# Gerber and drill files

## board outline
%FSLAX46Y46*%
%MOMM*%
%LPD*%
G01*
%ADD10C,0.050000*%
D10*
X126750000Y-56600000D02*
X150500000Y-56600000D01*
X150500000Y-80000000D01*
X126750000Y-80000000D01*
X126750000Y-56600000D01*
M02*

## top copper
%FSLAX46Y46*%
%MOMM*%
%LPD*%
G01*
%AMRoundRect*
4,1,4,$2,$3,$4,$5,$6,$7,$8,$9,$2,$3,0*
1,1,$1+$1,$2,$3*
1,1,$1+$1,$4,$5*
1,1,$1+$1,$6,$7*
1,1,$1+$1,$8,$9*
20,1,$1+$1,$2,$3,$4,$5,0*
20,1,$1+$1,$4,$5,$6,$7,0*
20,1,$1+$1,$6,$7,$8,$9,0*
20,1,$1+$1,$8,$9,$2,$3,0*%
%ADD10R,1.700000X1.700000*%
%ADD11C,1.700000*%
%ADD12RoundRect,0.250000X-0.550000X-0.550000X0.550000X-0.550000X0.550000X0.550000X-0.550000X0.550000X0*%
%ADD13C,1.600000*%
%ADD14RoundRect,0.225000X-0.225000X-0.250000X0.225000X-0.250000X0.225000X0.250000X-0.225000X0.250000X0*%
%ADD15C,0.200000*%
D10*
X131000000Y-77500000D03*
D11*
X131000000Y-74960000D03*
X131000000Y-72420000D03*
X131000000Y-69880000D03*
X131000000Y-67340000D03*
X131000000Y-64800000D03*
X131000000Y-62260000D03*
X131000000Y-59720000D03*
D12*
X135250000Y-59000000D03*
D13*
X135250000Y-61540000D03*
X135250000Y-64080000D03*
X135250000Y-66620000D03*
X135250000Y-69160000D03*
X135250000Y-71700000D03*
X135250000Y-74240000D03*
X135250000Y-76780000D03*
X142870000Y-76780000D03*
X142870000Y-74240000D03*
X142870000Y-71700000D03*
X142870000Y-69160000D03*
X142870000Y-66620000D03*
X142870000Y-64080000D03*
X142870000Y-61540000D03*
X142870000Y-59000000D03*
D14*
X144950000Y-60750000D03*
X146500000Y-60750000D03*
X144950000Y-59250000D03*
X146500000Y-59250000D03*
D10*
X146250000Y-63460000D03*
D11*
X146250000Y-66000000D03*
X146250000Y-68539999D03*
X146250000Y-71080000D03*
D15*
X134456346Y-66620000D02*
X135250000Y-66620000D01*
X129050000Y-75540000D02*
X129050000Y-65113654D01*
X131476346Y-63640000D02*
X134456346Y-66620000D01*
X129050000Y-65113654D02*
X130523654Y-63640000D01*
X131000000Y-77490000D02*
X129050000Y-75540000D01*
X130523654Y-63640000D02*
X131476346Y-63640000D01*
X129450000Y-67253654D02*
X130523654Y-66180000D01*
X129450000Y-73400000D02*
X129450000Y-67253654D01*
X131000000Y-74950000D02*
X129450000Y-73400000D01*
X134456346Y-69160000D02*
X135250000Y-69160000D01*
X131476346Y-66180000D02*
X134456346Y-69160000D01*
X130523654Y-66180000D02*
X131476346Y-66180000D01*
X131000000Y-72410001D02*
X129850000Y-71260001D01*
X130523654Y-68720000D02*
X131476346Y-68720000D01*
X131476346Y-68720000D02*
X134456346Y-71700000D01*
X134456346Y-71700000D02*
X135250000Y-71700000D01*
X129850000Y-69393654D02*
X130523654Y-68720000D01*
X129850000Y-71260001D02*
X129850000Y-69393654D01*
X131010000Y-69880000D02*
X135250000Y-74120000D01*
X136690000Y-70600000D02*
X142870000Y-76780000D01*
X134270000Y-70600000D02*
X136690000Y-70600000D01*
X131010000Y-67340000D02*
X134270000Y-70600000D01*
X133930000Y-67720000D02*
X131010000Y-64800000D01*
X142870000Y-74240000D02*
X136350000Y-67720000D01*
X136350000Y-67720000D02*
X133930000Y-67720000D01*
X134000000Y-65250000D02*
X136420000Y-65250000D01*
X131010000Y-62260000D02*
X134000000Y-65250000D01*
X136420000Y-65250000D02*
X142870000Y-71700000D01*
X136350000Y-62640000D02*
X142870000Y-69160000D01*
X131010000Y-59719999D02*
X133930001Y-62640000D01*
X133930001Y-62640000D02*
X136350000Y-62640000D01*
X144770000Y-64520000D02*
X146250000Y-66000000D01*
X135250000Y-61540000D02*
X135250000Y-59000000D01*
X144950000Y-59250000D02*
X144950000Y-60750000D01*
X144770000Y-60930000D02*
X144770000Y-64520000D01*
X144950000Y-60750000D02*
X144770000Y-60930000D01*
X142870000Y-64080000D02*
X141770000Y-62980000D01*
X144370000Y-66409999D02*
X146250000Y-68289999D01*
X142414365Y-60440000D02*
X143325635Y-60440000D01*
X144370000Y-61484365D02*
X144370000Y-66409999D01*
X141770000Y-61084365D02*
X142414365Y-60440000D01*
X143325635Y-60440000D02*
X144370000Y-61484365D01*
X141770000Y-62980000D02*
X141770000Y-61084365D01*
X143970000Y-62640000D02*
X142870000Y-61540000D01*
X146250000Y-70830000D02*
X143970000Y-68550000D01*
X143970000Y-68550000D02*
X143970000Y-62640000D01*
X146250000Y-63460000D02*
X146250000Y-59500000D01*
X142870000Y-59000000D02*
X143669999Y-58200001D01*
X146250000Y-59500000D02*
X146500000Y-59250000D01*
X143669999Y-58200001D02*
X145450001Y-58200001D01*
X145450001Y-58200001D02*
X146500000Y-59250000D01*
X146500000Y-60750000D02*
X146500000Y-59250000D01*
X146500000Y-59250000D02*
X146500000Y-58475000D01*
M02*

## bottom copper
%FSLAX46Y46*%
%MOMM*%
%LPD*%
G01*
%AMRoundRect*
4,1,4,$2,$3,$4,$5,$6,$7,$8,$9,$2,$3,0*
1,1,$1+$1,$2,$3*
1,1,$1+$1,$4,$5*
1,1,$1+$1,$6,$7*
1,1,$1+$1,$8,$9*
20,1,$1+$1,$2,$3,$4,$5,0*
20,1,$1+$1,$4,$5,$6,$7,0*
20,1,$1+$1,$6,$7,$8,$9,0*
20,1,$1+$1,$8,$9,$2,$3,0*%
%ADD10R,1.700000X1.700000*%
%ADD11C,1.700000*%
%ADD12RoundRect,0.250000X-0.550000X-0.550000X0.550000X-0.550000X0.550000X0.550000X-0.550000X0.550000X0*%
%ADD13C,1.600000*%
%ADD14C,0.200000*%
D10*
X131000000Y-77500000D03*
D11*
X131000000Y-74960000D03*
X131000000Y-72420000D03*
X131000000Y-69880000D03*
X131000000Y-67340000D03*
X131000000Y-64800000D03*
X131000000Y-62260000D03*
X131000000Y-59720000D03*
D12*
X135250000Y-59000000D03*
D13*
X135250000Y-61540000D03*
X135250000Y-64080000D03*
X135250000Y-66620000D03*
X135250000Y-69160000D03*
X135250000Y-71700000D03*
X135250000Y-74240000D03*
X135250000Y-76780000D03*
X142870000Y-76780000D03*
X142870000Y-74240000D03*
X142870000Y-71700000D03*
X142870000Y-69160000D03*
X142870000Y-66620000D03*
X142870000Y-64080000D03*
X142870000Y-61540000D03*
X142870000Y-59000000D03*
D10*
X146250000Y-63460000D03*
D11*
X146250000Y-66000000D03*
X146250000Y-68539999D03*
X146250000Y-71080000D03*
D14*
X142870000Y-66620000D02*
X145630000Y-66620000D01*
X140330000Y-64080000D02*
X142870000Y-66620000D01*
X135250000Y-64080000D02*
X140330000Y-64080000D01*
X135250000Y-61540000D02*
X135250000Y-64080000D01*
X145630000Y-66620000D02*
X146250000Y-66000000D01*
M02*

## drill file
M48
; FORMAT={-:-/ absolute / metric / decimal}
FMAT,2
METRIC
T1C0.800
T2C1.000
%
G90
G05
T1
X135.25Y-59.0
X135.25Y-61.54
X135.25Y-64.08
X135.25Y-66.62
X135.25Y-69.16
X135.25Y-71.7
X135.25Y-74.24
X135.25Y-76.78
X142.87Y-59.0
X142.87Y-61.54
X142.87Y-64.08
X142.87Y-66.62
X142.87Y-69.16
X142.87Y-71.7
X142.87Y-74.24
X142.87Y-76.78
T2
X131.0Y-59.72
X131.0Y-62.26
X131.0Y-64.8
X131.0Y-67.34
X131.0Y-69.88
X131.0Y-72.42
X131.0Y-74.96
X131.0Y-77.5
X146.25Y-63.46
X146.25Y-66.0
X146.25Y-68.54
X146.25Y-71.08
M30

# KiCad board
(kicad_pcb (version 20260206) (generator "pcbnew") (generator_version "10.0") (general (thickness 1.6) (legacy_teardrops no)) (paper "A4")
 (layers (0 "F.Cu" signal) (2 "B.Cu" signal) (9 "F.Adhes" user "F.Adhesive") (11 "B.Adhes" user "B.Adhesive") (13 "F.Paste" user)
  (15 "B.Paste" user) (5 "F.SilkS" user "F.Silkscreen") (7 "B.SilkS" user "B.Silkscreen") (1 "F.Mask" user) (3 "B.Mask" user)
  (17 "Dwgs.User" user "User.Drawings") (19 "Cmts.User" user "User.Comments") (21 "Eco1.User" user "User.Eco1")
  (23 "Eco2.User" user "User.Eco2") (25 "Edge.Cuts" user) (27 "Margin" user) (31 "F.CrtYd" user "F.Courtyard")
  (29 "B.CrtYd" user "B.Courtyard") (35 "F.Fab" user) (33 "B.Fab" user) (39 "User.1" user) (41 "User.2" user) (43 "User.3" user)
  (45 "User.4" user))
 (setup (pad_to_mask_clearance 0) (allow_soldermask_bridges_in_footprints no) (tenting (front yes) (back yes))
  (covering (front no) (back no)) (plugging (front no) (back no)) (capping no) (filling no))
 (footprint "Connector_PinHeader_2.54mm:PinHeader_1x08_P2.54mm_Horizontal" (layer "F.Cu") (at 131 77.5 180)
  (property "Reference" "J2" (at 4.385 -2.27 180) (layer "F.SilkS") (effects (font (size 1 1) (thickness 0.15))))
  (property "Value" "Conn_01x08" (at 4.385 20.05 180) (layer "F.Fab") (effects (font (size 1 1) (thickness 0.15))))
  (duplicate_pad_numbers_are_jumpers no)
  (pad "1" thru_hole rect (at 0 0 180) (size 1.7 1.7) (drill 1) (layers "*.Cu" "*.Mask") (remove_unused_layers no) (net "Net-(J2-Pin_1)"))
  (pad "2" thru_hole circle (at 0 2.54 180) (size 1.7 1.7) (drill 1) (layers "*.Cu" "*.Mask") (remove_unused_layers no)
   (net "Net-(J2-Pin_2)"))
  (pad "3" thru_hole circle (at 0 5.08 180) (size 1.7 1.7) (drill 1) (layers "*.Cu" "*.Mask") (remove_unused_layers no)
   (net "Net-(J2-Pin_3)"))
  (pad "4" thru_hole circle (at 0 7.62 180) (size 1.7 1.7) (drill 1) (layers "*.Cu" "*.Mask") (remove_unused_layers no)
   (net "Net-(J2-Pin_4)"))
  (pad "5" thru_hole circle (at 0 10.16 180) (size 1.7 1.7) (drill 1) (layers "*.Cu" "*.Mask") (remove_unused_layers no)
   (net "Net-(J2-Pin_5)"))
  (pad "6" thru_hole circle (at 0 12.7 180) (size 1.7 1.7) (drill 1) (layers "*.Cu" "*.Mask") (remove_unused_layers no)
   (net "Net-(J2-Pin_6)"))
  (pad "7" thru_hole circle (at 0 15.24 180) (size 1.7 1.7) (drill 1) (layers "*.Cu" "*.Mask") (remove_unused_layers no)
   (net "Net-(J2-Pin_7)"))
  (pad "8" thru_hole circle (at 0 17.78 180) (size 1.7 1.7) (drill 1) (layers "*.Cu" "*.Mask") (remove_unused_layers no)
   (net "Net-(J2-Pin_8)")))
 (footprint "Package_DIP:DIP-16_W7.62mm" (layer "F.Cu") (at 135.25 59)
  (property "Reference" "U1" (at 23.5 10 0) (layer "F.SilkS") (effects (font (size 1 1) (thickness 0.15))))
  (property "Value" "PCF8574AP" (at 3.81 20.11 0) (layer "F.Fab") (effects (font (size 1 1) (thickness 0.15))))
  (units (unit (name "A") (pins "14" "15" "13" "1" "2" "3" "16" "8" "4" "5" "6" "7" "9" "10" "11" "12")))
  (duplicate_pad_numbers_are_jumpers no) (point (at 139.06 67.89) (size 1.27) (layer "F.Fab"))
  (pad "1" thru_hole roundrect (at 0 0) (size 1.6 1.6) (drill 0.8) (layers "*.Cu" "*.Mask") (remove_unused_layers no)
   (roundrect_rratio 0.15625) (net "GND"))
  (pad "2" thru_hole circle (at 0 2.54) (size 1.6 1.6) (drill 0.8) (layers "*.Cu" "*.Mask") (remove_unused_layers no) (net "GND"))
  (pad "3" thru_hole circle (at 0 5.08) (size 1.6 1.6) (drill 0.8) (layers "*.Cu" "*.Mask") (remove_unused_layers no) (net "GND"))
  (pad "4" thru_hole circle (at 0 7.62) (size 1.6 1.6) (drill 0.8) (layers "*.Cu" "*.Mask") (remove_unused_layers no) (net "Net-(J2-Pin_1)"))
  (pad "5" thru_hole circle (at 0 10.16) (size 1.6 1.6) (drill 0.8) (layers "*.Cu" "*.Mask") (remove_unused_layers no)
   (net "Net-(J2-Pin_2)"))
  (pad "6" thru_hole circle (at 0 12.7) (size 1.6 1.6) (drill 0.8) (layers "*.Cu" "*.Mask") (remove_unused_layers no) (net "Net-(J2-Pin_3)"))
  (pad "7" thru_hole circle (at 0 15.24) (size 1.6 1.6) (drill 0.8) (layers "*.Cu" "*.Mask") (remove_unused_layers no)
   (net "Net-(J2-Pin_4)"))
  (pad "8" thru_hole circle (at 0 17.78) (size 1.6 1.6) (drill 0.8) (layers "*.Cu" "*.Mask") (remove_unused_layers no)
   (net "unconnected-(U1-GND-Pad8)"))
  (pad "9" thru_hole circle (at 7.62 17.78) (size 1.6 1.6) (drill 0.8) (layers "*.Cu" "*.Mask") (remove_unused_layers no)
   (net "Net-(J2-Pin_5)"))
  (pad "10" thru_hole circle (at 7.62 15.24) (size 1.6 1.6) (drill 0.8) (layers "*.Cu" "*.Mask") (remove_unused_layers no)
   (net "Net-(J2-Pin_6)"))
  (pad "11" thru_hole circle (at 7.62 12.7) (size 1.6 1.6) (drill 0.8) (layers "*.Cu" "*.Mask") (remove_unused_layers no)
   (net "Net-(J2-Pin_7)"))
  (pad "12" thru_hole circle (at 7.62 10.16) (size 1.6 1.6) (drill 0.8) (layers "*.Cu" "*.Mask") (remove_unused_layers no)
   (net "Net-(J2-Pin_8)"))
  (pad "13" thru_hole circle (at 7.62 7.62) (size 1.6 1.6) (drill 0.8) (layers "*.Cu" "*.Mask") (remove_unused_layers no) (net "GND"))
  (pad "14" thru_hole circle (at 7.62 5.08) (size 1.6 1.6) (drill 0.8) (layers "*.Cu" "*.Mask") (remove_unused_layers no) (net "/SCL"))
  (pad "15" thru_hole circle (at 7.62 2.54) (size 1.6 1.6) (drill 0.8) (layers "*.Cu" "*.Mask") (remove_unused_layers no) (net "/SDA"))
  (pad "16" thru_hole circle (at 7.62 0) (size 1.6 1.6) (drill 0.8) (layers "*.Cu" "*.Mask") (remove_unused_layers no) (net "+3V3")))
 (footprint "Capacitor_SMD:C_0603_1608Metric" (layer "F.Cu") (at 145.725 60.75)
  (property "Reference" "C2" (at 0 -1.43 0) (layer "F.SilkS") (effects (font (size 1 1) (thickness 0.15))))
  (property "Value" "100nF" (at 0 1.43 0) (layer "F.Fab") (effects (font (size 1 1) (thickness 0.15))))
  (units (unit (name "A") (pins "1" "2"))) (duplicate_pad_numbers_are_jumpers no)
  (pad "1" smd roundrect (at -0.775 0) (size 0.9 0.95) (layers "F.Cu" "F.Mask" "F.Paste") (roundrect_rratio 0.25) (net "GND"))
  (pad "2" smd roundrect (at 0.775 0) (size 0.9 0.95) (layers "F.Cu" "F.Mask" "F.Paste") (roundrect_rratio 0.25) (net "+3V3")))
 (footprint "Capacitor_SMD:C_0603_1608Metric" (layer "F.Cu") (at 145.725 59.25)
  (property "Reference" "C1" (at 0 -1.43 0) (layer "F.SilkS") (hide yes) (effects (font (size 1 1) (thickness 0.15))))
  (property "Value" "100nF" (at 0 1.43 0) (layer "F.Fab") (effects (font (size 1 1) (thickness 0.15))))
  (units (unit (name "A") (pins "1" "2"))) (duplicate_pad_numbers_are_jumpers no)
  (pad "1" smd roundrect (at -0.775 0) (size 0.9 0.95) (layers "F.Cu" "F.Mask" "F.Paste") (roundrect_rratio 0.25) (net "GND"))
  (pad "2" smd roundrect (at 0.775 0) (size 0.9 0.95) (layers "F.Cu" "F.Mask" "F.Paste") (roundrect_rratio 0.25) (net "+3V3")))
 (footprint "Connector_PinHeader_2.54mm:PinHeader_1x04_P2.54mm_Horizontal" (layer "F.Cu") (at 146.25 63.46)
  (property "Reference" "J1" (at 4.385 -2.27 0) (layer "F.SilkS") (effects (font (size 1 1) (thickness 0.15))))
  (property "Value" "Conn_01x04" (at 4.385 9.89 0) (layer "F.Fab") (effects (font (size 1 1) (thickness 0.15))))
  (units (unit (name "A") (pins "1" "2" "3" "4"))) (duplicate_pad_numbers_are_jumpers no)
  (pad "1" thru_hole rect (at 0 0) (size 1.7 1.7) (drill 1) (layers "*.Cu" "*.Mask") (remove_unused_layers no) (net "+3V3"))
  (pad "2" thru_hole circle (at 0 2.54) (size 1.7 1.7) (drill 1) (layers "*.Cu" "*.Mask") (remove_unused_layers no) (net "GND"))
  (pad "3" thru_hole circle (at 0 5.079999) (size 1.7 1.7) (drill 1) (layers "*.Cu" "*.Mask") (remove_unused_layers no) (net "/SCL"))
  (pad "4" thru_hole circle (at 0 7.62) (size 1.7 1.7) (drill 1) (layers "*.Cu" "*.Mask") (remove_unused_layers no) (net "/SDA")))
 (gr_rect (start 126.75 56.6) (end 150.5 80) (stroke (width 0.05) (type default)) (fill no) (layer "Edge.Cuts"))
 (segment (start 134.456346 66.62) (end 135.25 66.62) (width 0.2) (layer "F.Cu") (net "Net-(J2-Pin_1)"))
 (segment (start 129.05 75.54) (end 129.05 65.113654) (width 0.2) (layer "F.Cu") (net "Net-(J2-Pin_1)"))
 (segment (start 131.476346 63.64) (end 134.456346 66.62) (width 0.2) (layer "F.Cu") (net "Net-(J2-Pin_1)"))
 (segment (start 129.05 65.113654) (end 130.523654 63.64) (width 0.2) (layer "F.Cu") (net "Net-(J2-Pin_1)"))
 (segment (start 131 77.49) (end 129.05 75.54) (width 0.2) (layer "F.Cu") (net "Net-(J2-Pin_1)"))
 (segment (start 130.523654 63.64) (end 131.476346 63.64) (width 0.2) (layer "F.Cu") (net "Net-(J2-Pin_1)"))
 (segment (start 129.45 67.253654) (end 130.523654 66.18) (width 0.2) (layer "F.Cu") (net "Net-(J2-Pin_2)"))
 (segment (start 129.45 73.4) (end 129.45 67.253654) (width 0.2) (layer "F.Cu") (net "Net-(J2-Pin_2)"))
 (segment (start 131 74.95) (end 129.45 73.4) (width 0.2) (layer "F.Cu") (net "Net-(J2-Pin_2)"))
 (segment (start 134.456346 69.16) (end 135.25 69.16) (width 0.2) (layer "F.Cu") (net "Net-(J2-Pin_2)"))
 (segment (start 131.476346 66.18) (end 134.456346 69.16) (width 0.2) (layer "F.Cu") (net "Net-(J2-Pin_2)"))
 (segment (start 130.523654 66.18) (end 131.476346 66.18) (width 0.2) (layer "F.Cu") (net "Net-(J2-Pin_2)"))
 (segment (start 131 72.410001) (end 129.85 71.260001) (width 0.2) (layer "F.Cu") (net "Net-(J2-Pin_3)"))
 (segment (start 130.523654 68.72) (end 131.476346 68.72) (width 0.2) (layer "F.Cu") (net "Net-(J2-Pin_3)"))
 (segment (start 131.476346 68.72) (end 134.456346 71.7) (width 0.2) (layer "F.Cu") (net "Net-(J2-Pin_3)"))
 (segment (start 134.456346 71.7) (end 135.25 71.7) (width 0.2) (layer "F.Cu") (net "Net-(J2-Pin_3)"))
 (segment (start 129.85 69.393654) (end 130.523654 68.72) (width 0.2) (layer "F.Cu") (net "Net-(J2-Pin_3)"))
 (segment (start 129.85 71.260001) (end 129.85 69.393654) (width 0.2) (layer "F.Cu") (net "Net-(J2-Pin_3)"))
 (segment (start 131.01 69.88) (end 135.25 74.12) (width 0.2) (layer "F.Cu") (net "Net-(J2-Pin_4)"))
 (segment (start 136.69 70.6) (end 142.87 76.78) (width 0.2) (layer "F.Cu") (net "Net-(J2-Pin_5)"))
 (segment (start 134.27 70.6) (end 136.69 70.6) (width 0.2) (layer "F.Cu") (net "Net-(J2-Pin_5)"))
 (segment (start 131.01 67.34) (end 134.27 70.6) (width 0.2) (layer "F.Cu") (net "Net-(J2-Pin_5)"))
 (segment (start 133.93 67.72) (end 131.01 64.8) (width 0.2) (layer "F.Cu") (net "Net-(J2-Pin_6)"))
 (segment (start 142.87 74.24) (end 136.35 67.72) (width 0.2) (layer "F.Cu") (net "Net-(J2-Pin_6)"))
 (segment (start 136.35 67.72) (end 133.93 67.72) (width 0.2) (layer "F.Cu") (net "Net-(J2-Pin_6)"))
 (segment (start 134 65.25) (end 136.42 65.25) (width 0.2) (layer "F.Cu") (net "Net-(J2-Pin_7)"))
 (segment (start 131.01 62.26) (end 134 65.25) (width 0.2) (layer "F.Cu") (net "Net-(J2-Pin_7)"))
 (segment (start 136.42 65.25) (end 142.87 71.7) (width 0.2) (layer "F.Cu") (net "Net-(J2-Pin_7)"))
 (segment (start 136.35 62.64) (end 142.87 69.16) (width 0.2) (layer "F.Cu") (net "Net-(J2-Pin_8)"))
 (segment (start 131.01 59.719999) (end 133.930001 62.64) (width 0.2) (layer "F.Cu") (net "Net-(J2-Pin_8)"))
 (segment (start 133.930001 62.64) (end 136.35 62.64) (width 0.2) (layer "F.Cu") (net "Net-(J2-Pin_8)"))
 (segment (start 144.77 64.52) (end 146.25 66) (width 0.2) (layer "F.Cu") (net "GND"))
 (segment (start 135.25 61.54) (end 135.25 59) (width 0.2) (layer "F.Cu") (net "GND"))
 (segment (start 144.95 59.25) (end 144.95 60.75) (width 0.2) (layer "F.Cu") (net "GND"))
 (segment (start 144.77 60.93) (end 144.77 64.52) (width 0.2) (layer "F.Cu") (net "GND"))
 (segment (start 144.95 60.75) (end 144.77 60.93) (width 0.2) (layer "F.Cu") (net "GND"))
 (segment (start 142.87 66.62) (end 145.63 66.62) (width 0.2) (layer "B.Cu") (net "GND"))
 (segment (start 140.33 64.08) (end 142.87 66.62) (width 0.2) (layer "B.Cu") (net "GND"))
 (segment (start 135.25 64.08) (end 140.33 64.08) (width 0.2) (layer "B.Cu") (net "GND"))
 (segment (start 135.25 61.54) (end 135.25 64.08) (width 0.2) (layer "B.Cu") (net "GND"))
 (segment (start 145.63 66.62) (end 146.25 66) (width 0.2) (layer "B.Cu") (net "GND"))
 (segment (start 142.87 64.08) (end 141.77 62.98) (width 0.2) (layer "F.Cu") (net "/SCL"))
 (segment (start 144.37 66.409999) (end 146.25 68.289999) (width 0.2) (layer "F.Cu") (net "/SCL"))
 (segment (start 142.414365 60.44) (end 143.325635 60.44) (width 0.2) (layer "F.Cu") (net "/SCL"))
 (segment (start 144.37 61.484365) (end 144.37 66.409999) (width 0.2) (layer "F.Cu") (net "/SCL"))
 (segment (start 141.77 61.084365) (end 142.414365 60.44) (width 0.2) (layer "F.Cu") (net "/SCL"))
 (segment (start 143.325635 60.44) (end 144.37 61.484365) (width 0.2) (layer "F.Cu") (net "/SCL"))
 (segment (start 141.77 62.98) (end 141.77 61.084365) (width 0.2) (layer "F.Cu") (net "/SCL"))
 (segment (start 143.97 62.64) (end 142.87 61.54) (width 0.2) (layer "F.Cu") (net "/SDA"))
 (segment (start 146.25 70.83) (end 143.97 68.55) (width 0.2) (layer "F.Cu") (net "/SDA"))
 (segment (start 143.97 68.55) (end 143.97 62.64) (width 0.2) (layer "F.Cu") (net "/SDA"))
 (segment (start 146.25 63.46) (end 146.25 59.5) (width 0.2) (layer "F.Cu") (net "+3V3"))
 (segment (start 142.87 59) (end 143.669999 58.200001) (width 0.2) (layer "F.Cu") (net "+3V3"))
 (segment (start 146.25 59.5) (end 146.5 59.25) (width 0.2) (layer "F.Cu") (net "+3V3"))
 (segment (start 143.669999 58.200001) (end 145.450001 58.200001) (width 0.2) (layer "F.Cu") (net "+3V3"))
 (segment (start 145.450001 58.200001) (end 146.5 59.25) (width 0.2) (layer "F.Cu") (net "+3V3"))
 (segment (start 146.5 60.75) (end 146.5 59.25) (width 0.2) (layer "F.Cu") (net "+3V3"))
 (segment (start 146.5 59.25) (end 146.5 58.475) (width 0.2) (layer "F.Cu") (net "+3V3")))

